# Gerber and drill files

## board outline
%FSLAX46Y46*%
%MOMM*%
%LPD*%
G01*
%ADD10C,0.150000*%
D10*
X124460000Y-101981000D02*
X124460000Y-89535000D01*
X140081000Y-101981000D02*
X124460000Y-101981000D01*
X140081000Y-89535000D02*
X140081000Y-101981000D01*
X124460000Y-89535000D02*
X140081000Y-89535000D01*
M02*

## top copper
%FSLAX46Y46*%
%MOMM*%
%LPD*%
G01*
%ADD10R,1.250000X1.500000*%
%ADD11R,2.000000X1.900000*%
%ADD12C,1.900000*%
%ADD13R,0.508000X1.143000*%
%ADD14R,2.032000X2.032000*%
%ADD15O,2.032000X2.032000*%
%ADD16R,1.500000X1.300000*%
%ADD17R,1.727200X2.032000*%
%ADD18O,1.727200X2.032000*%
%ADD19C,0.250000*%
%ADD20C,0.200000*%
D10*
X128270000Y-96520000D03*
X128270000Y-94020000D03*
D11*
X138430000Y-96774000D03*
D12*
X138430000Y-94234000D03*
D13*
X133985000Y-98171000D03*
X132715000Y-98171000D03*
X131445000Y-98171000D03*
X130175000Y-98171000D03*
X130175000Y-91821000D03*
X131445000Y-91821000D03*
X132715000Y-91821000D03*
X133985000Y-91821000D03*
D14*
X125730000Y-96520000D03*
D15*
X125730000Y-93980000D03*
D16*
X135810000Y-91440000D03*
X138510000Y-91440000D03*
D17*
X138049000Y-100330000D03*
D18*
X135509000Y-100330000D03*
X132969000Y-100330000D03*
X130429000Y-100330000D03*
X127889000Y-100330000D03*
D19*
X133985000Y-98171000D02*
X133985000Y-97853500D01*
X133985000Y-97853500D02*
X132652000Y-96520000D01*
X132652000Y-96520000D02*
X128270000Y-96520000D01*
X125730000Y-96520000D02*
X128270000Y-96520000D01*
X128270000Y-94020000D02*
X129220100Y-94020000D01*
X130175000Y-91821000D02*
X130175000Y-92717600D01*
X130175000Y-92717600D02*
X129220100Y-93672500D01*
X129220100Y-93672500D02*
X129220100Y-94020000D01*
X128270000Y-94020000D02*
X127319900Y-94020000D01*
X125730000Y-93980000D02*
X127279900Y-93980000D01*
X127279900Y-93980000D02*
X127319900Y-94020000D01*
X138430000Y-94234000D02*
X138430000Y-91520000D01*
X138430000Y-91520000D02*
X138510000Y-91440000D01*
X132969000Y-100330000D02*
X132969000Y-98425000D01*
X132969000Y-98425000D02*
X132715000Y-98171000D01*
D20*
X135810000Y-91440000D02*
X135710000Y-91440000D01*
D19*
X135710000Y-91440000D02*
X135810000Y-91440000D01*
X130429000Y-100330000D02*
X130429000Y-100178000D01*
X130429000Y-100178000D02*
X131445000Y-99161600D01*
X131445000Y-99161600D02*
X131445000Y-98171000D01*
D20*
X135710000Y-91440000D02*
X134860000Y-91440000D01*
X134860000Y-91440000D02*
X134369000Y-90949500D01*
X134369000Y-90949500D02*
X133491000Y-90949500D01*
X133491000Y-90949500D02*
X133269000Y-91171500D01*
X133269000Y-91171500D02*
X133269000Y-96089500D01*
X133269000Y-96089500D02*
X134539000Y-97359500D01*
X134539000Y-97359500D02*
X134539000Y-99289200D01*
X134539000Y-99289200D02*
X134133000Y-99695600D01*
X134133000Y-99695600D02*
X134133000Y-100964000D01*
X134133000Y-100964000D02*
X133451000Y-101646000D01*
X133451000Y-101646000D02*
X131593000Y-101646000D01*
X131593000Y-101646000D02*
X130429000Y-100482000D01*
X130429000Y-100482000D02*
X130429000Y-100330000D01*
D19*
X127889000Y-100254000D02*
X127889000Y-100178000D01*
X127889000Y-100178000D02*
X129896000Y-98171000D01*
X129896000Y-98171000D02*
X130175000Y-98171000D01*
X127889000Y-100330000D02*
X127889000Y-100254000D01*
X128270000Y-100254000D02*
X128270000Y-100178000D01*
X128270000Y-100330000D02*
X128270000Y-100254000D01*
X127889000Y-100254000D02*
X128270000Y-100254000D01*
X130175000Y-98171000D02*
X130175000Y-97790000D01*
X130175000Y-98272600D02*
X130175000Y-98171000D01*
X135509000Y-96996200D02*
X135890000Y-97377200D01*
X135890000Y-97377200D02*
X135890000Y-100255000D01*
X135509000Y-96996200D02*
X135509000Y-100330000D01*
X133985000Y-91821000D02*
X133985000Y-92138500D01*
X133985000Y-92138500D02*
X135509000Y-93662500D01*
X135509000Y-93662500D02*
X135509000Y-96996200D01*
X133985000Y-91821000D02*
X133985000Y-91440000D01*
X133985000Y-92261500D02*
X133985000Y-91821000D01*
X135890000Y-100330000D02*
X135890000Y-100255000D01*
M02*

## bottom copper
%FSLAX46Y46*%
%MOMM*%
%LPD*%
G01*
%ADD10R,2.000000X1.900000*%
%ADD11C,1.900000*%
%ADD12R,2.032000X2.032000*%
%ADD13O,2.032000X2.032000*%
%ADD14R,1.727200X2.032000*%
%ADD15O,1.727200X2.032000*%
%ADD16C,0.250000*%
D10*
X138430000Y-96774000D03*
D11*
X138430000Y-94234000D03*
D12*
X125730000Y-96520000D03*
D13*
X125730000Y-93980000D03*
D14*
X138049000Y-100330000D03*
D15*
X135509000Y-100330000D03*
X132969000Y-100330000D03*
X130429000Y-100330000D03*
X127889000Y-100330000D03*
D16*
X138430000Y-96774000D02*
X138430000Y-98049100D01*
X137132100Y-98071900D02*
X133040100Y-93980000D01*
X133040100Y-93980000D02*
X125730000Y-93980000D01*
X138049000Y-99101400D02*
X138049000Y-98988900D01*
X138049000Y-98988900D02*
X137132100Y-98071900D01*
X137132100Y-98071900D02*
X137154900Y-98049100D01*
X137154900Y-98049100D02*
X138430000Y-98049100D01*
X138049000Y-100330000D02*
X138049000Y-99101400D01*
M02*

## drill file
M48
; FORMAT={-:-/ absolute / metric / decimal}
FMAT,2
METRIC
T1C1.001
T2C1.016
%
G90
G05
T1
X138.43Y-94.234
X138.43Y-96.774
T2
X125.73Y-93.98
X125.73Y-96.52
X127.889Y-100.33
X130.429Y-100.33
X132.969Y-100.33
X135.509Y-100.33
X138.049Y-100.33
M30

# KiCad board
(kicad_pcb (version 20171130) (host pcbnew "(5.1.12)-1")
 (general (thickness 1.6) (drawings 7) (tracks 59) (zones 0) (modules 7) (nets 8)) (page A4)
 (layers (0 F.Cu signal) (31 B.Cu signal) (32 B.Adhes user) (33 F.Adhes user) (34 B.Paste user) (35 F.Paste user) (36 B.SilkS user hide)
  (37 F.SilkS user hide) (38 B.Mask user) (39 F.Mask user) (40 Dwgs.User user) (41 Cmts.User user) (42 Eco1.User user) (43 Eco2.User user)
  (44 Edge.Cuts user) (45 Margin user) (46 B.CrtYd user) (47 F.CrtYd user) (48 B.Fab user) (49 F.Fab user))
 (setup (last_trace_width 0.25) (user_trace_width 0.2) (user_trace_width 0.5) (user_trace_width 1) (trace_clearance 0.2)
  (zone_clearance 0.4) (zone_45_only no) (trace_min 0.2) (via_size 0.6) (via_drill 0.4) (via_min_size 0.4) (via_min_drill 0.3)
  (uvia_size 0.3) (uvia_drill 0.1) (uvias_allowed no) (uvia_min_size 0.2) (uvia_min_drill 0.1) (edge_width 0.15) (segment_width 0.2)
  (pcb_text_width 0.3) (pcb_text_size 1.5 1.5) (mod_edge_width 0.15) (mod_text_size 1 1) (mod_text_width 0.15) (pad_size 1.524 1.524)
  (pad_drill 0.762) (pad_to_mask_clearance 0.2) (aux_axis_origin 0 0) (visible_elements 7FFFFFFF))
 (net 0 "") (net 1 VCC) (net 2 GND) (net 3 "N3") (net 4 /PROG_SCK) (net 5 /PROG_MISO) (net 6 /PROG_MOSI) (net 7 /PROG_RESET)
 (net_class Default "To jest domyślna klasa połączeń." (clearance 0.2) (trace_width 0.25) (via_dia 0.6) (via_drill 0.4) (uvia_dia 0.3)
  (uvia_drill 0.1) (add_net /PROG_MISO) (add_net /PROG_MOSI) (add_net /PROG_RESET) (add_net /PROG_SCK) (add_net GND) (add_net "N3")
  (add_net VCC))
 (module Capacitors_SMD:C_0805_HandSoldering (layer F.Cu) (at 128.27 95.27 90)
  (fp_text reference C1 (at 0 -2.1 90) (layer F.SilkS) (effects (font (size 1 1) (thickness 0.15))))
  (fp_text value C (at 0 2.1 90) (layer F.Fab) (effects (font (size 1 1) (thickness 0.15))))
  (pad 1 smd rect (at -1.25 0 90) (size 1.5 1.25) (layers F.Cu F.Paste F.Mask) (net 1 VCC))
  (pad 2 smd rect (at 1.25 0 90) (size 1.5 1.25) (layers F.Cu F.Paste F.Mask) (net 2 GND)))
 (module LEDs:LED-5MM (layer B.Cu) (at 138.43 96.774 90)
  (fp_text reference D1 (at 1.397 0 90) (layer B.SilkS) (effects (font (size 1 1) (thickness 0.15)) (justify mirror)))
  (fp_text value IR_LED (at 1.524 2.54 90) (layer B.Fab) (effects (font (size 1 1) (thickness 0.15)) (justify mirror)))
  (pad 1 thru_hole rect (at 0 0) (size 2 1.9) (drill 1.00076) (layers *.Cu *.Mask B.SilkS) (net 2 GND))
  (pad 2 thru_hole circle (at 2.54 0 90) (size 1.9 1.9) (drill 1.00076) (layers *.Cu *.Mask B.SilkS) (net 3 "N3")))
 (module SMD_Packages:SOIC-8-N (layer F.Cu) (at 132.08 94.996 180)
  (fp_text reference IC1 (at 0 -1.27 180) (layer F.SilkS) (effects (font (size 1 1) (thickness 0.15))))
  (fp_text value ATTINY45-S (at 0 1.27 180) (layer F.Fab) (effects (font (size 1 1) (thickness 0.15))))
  (pad 8 smd rect (at -1.905 -3.175 180) (size 0.508 1.143) (layers F.Cu F.Paste F.Mask) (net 1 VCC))
  (pad 7 smd rect (at -0.635 -3.175 180) (size 0.508 1.143) (layers F.Cu F.Paste F.Mask) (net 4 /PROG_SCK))
  (pad 6 smd rect (at 0.635 -3.175 180) (size 0.508 1.143) (layers F.Cu F.Paste F.Mask) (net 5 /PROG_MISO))
  (pad 5 smd rect (at 1.905 -3.175 180) (size 0.508 1.143) (layers F.Cu F.Paste F.Mask) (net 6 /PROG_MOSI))
  (pad 4 smd rect (at 1.905 3.175 180) (size 0.508 1.143) (layers F.Cu F.Paste F.Mask) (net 2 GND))
  (pad 3 smd rect (at 0.635 3.175 180) (size 0.508 1.143) (layers F.Cu F.Paste F.Mask))
  (pad 2 smd rect (at -0.635 3.175 180) (size 0.508 1.143) (layers F.Cu F.Paste F.Mask))
  (pad 1 smd rect (at -1.905 3.175 180) (size 0.508 1.143) (layers F.Cu F.Paste F.Mask) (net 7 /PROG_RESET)))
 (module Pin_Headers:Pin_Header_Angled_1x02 (layer F.Cu) (at 125.73 96.52 180)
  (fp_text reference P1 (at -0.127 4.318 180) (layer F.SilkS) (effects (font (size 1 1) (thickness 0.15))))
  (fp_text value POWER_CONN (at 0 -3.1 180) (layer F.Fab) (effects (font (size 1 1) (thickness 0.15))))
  (pad 1 thru_hole rect (at 0 0 180) (size 2.032 2.032) (drill 1.016) (layers *.Cu *.Mask F.SilkS) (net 1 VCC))
  (pad 2 thru_hole oval (at 0 2.54 180) (size 2.032 2.032) (drill 1.016) (layers *.Cu *.Mask F.SilkS) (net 2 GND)))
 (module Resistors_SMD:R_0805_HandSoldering (layer F.Cu) (at 137.16 91.44)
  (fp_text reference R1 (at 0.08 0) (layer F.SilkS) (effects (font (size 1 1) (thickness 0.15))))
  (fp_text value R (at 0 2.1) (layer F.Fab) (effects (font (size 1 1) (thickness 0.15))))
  (pad 1 smd rect (at -1.35 0) (size 1.5 1.3) (layers F.Cu F.Paste F.Mask) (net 5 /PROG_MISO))
  (pad 2 smd rect (at 1.35 0) (size 1.5 1.3) (layers F.Cu F.Paste F.Mask) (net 3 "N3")))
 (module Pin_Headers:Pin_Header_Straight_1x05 (layer F.Cu) (at 138.049 100.33 270)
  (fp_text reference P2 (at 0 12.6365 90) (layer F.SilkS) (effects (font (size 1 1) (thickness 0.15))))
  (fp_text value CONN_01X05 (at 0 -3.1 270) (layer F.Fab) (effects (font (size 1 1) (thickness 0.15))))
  (pad 1 thru_hole rect (at 0 0 270) (size 2.032 1.7272) (drill 1.016) (layers *.Cu *.Mask F.SilkS) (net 2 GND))
  (pad 2 thru_hole oval (at 0 2.54 270) (size 2.032 1.7272) (drill 1.016) (layers *.Cu *.Mask F.SilkS) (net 7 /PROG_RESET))
  (pad 3 thru_hole oval (at 0 5.08 270) (size 2.032 1.7272) (drill 1.016) (layers *.Cu *.Mask F.SilkS) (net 4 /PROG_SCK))
  (pad 4 thru_hole oval (at 0 7.62 270) (size 2.032 1.7272) (drill 1.016) (layers *.Cu *.Mask F.SilkS) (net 5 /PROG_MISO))
  (pad 5 thru_hole oval (at 0 10.16 270) (size 2.032 1.7272) (drill 1.016) (layers *.Cu *.Mask F.SilkS) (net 6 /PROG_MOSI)))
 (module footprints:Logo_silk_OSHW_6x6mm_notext (layer B.Cu) (at 129.794 92.202)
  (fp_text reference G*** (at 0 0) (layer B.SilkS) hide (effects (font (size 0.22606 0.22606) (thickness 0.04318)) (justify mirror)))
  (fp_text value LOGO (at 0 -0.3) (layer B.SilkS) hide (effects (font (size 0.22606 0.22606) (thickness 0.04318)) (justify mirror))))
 (gr_line (start 124.46 101.981) (end 124.46 89.535) (layer Edge.Cuts) (width 0.15))
 (gr_line (start 140.081 101.981) (end 124.46 101.981) (layer Edge.Cuts) (width 0.15))
 (gr_line (start 140.081 89.535) (end 140.081 101.981) (layer Edge.Cuts) (width 0.15))
 (gr_line (start 124.46 89.535) (end 140.081 89.535) (layer Edge.Cuts) (width 0.15))
 (segment (start 133.985 98.171) (end 133.985 97.8535) (width 0.25) (layer F.Cu) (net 1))
 (segment (start 133.985 97.8535) (end 132.652 96.52) (width 0.25) (layer F.Cu) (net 1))
 (segment (start 132.652 96.52) (end 128.27 96.52) (width 0.25) (layer F.Cu) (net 1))
 (segment (start 125.73 96.52) (end 128.27 96.52) (width 0.25) (layer F.Cu) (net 1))
 (segment (start 138.43 96.774) (end 138.43 98.0491) (width 0.25) (layer B.Cu) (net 2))
 (segment (start 137.1321 98.0719) (end 133.0401 93.98) (width 0.25) (layer B.Cu) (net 2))
 (segment (start 133.0401 93.98) (end 125.73 93.98) (width 0.25) (layer B.Cu) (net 2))
 (segment (start 138.049 99.1014) (end 138.049 98.9889) (width 0.25) (layer B.Cu) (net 2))
 (segment (start 138.049 98.9889) (end 137.1321 98.0719) (width 0.25) (layer B.Cu) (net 2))
 (segment (start 137.1321 98.0719) (end 137.1549 98.0491) (width 0.25) (layer B.Cu) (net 2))
 (segment (start 137.1549 98.0491) (end 138.43 98.0491) (width 0.25) (layer B.Cu) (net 2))
 (segment (start 138.049 100.33) (end 138.049 99.1014) (width 0.25) (layer B.Cu) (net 2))
 (segment (start 128.27 94.02) (end 129.2201 94.02) (width 0.25) (layer F.Cu) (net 2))
 (segment (start 130.175 91.821) (end 130.175 92.7176) (width 0.25) (layer F.Cu) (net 2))
 (segment (start 130.175 92.7176) (end 129.2201 93.6725) (width 0.25) (layer F.Cu) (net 2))
 (segment (start 129.2201 93.6725) (end 129.2201 94.02) (width 0.25) (layer F.Cu) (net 2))
 (segment (start 128.27 94.02) (end 127.3199 94.02) (width 0.25) (layer F.Cu) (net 2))
 (segment (start 125.73 93.98) (end 127.2799 93.98) (width 0.25) (layer F.Cu) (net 2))
 (segment (start 127.2799 93.98) (end 127.3199 94.02) (width 0.25) (layer F.Cu) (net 2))
 (segment (start 138.43 94.234) (end 138.43 91.52) (width 0.25) (layer F.Cu) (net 3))
 (segment (start 138.43 91.52) (end 138.51 91.44) (width 0.25) (layer F.Cu) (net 3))
 (segment (start 132.969 100.33) (end 132.969 98.425) (width 0.25) (layer F.Cu) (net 4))
 (segment (start 132.969 98.425) (end 132.715 98.171) (width 0.25) (layer F.Cu) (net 4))
 (segment (start 135.81 91.44) (end 135.71 91.44) (width 0.2) (layer F.Cu) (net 5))
 (segment (start 135.71 91.44) (end 135.81 91.44) (width 0.25) (layer F.Cu) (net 5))
 (segment (start 130.429 100.33) (end 130.429 100.178) (width 0.25) (layer F.Cu) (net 5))
 (segment (start 130.429 100.178) (end 131.445 99.1616) (width 0.25) (layer F.Cu) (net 5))
 (segment (start 131.445 99.1616) (end 131.445 98.171) (width 0.25) (layer F.Cu) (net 5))
 (segment (start 135.71 91.44) (end 134.86 91.44) (width 0.2) (layer F.Cu) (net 5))
 (segment (start 134.86 91.44) (end 134.369 90.9495) (width 0.2) (layer F.Cu) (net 5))
 (segment (start 134.369 90.9495) (end 133.491 90.9495) (width 0.2) (layer F.Cu) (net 5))
 (segment (start 133.491 90.9495) (end 133.269 91.1715) (width 0.2) (layer F.Cu) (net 5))
 (segment (start 133.269 91.1715) (end 133.269 96.0895) (width 0.2) (layer F.Cu) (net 5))
 (segment (start 133.269 96.0895) (end 134.539 97.3595) (width 0.2) (layer F.Cu) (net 5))
 (segment (start 134.539 97.3595) (end 134.539 99.2892) (width 0.2) (layer F.Cu) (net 5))
 (segment (start 134.539 99.2892) (end 134.133 99.6956) (width 0.2) (layer F.Cu) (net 5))
 (segment (start 134.133 99.6956) (end 134.133 100.964) (width 0.2) (layer F.Cu) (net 5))
 (segment (start 134.133 100.964) (end 133.451 101.646) (width 0.2) (layer F.Cu) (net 5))
 (segment (start 133.451 101.646) (end 131.593 101.646) (width 0.2) (layer F.Cu) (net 5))
 (segment (start 131.593 101.646) (end 130.429 100.482) (width 0.2) (layer F.Cu) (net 5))
 (segment (start 130.429 100.482) (end 130.429 100.33) (width 0.2) (layer F.Cu) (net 5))
 (segment (start 127.889 100.254) (end 127.889 100.178) (width 0.25) (layer F.Cu) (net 6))
 (segment (start 127.889 100.178) (end 129.896 98.171) (width 0.25) (layer F.Cu) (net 6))
 (segment (start 129.896 98.171) (end 130.175 98.171) (width 0.25) (layer F.Cu) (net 6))
 (segment (start 127.889 100.33) (end 127.889 100.254) (width 0.25) (layer F.Cu) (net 6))
 (segment (start 128.27 100.254) (end 128.27 100.178) (width 0.25) (layer F.Cu) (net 6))
 (segment (start 128.27 100.33) (end 128.27 100.254) (width 0.25) (layer F.Cu) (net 6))
 (segment (start 127.889 100.254) (end 128.27 100.254) (width 0.25) (layer F.Cu) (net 6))
 (segment (start 130.175 98.171) (end 130.175 97.79) (width 0.25) (layer F.Cu) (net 6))
 (segment (start 130.175 98.2726) (end 130.175 98.171) (width 0.25) (layer F.Cu) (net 6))
 (segment (start 135.509 96.9962) (end 135.89 97.3772) (width 0.25) (layer F.Cu) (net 7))
 (segment (start 135.89 97.3772) (end 135.89 100.255) (width 0.25) (layer F.Cu) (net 7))
 (segment (start 135.509 96.9962) (end 135.509 100.33) (width 0.25) (layer F.Cu) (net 7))
 (segment (start 133.985 91.821) (end 133.985 92.1385) (width 0.25) (layer F.Cu) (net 7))
 (segment (start 133.985 92.1385) (end 135.509 93.6625) (width 0.25) (layer F.Cu) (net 7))
 (segment (start 135.509 93.6625) (end 135.509 96.9962) (width 0.25) (layer F.Cu) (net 7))
 (segment (start 133.985 91.821) (end 133.985 91.44) (width 0.25) (layer F.Cu) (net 7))
 (segment (start 133.985 92.2615) (end 133.985 91.821) (width 0.25) (layer F.Cu) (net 7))
 (segment (start 135.89 100.33) (end 135.89 100.255) (width 0.25) (layer F.Cu) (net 7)))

